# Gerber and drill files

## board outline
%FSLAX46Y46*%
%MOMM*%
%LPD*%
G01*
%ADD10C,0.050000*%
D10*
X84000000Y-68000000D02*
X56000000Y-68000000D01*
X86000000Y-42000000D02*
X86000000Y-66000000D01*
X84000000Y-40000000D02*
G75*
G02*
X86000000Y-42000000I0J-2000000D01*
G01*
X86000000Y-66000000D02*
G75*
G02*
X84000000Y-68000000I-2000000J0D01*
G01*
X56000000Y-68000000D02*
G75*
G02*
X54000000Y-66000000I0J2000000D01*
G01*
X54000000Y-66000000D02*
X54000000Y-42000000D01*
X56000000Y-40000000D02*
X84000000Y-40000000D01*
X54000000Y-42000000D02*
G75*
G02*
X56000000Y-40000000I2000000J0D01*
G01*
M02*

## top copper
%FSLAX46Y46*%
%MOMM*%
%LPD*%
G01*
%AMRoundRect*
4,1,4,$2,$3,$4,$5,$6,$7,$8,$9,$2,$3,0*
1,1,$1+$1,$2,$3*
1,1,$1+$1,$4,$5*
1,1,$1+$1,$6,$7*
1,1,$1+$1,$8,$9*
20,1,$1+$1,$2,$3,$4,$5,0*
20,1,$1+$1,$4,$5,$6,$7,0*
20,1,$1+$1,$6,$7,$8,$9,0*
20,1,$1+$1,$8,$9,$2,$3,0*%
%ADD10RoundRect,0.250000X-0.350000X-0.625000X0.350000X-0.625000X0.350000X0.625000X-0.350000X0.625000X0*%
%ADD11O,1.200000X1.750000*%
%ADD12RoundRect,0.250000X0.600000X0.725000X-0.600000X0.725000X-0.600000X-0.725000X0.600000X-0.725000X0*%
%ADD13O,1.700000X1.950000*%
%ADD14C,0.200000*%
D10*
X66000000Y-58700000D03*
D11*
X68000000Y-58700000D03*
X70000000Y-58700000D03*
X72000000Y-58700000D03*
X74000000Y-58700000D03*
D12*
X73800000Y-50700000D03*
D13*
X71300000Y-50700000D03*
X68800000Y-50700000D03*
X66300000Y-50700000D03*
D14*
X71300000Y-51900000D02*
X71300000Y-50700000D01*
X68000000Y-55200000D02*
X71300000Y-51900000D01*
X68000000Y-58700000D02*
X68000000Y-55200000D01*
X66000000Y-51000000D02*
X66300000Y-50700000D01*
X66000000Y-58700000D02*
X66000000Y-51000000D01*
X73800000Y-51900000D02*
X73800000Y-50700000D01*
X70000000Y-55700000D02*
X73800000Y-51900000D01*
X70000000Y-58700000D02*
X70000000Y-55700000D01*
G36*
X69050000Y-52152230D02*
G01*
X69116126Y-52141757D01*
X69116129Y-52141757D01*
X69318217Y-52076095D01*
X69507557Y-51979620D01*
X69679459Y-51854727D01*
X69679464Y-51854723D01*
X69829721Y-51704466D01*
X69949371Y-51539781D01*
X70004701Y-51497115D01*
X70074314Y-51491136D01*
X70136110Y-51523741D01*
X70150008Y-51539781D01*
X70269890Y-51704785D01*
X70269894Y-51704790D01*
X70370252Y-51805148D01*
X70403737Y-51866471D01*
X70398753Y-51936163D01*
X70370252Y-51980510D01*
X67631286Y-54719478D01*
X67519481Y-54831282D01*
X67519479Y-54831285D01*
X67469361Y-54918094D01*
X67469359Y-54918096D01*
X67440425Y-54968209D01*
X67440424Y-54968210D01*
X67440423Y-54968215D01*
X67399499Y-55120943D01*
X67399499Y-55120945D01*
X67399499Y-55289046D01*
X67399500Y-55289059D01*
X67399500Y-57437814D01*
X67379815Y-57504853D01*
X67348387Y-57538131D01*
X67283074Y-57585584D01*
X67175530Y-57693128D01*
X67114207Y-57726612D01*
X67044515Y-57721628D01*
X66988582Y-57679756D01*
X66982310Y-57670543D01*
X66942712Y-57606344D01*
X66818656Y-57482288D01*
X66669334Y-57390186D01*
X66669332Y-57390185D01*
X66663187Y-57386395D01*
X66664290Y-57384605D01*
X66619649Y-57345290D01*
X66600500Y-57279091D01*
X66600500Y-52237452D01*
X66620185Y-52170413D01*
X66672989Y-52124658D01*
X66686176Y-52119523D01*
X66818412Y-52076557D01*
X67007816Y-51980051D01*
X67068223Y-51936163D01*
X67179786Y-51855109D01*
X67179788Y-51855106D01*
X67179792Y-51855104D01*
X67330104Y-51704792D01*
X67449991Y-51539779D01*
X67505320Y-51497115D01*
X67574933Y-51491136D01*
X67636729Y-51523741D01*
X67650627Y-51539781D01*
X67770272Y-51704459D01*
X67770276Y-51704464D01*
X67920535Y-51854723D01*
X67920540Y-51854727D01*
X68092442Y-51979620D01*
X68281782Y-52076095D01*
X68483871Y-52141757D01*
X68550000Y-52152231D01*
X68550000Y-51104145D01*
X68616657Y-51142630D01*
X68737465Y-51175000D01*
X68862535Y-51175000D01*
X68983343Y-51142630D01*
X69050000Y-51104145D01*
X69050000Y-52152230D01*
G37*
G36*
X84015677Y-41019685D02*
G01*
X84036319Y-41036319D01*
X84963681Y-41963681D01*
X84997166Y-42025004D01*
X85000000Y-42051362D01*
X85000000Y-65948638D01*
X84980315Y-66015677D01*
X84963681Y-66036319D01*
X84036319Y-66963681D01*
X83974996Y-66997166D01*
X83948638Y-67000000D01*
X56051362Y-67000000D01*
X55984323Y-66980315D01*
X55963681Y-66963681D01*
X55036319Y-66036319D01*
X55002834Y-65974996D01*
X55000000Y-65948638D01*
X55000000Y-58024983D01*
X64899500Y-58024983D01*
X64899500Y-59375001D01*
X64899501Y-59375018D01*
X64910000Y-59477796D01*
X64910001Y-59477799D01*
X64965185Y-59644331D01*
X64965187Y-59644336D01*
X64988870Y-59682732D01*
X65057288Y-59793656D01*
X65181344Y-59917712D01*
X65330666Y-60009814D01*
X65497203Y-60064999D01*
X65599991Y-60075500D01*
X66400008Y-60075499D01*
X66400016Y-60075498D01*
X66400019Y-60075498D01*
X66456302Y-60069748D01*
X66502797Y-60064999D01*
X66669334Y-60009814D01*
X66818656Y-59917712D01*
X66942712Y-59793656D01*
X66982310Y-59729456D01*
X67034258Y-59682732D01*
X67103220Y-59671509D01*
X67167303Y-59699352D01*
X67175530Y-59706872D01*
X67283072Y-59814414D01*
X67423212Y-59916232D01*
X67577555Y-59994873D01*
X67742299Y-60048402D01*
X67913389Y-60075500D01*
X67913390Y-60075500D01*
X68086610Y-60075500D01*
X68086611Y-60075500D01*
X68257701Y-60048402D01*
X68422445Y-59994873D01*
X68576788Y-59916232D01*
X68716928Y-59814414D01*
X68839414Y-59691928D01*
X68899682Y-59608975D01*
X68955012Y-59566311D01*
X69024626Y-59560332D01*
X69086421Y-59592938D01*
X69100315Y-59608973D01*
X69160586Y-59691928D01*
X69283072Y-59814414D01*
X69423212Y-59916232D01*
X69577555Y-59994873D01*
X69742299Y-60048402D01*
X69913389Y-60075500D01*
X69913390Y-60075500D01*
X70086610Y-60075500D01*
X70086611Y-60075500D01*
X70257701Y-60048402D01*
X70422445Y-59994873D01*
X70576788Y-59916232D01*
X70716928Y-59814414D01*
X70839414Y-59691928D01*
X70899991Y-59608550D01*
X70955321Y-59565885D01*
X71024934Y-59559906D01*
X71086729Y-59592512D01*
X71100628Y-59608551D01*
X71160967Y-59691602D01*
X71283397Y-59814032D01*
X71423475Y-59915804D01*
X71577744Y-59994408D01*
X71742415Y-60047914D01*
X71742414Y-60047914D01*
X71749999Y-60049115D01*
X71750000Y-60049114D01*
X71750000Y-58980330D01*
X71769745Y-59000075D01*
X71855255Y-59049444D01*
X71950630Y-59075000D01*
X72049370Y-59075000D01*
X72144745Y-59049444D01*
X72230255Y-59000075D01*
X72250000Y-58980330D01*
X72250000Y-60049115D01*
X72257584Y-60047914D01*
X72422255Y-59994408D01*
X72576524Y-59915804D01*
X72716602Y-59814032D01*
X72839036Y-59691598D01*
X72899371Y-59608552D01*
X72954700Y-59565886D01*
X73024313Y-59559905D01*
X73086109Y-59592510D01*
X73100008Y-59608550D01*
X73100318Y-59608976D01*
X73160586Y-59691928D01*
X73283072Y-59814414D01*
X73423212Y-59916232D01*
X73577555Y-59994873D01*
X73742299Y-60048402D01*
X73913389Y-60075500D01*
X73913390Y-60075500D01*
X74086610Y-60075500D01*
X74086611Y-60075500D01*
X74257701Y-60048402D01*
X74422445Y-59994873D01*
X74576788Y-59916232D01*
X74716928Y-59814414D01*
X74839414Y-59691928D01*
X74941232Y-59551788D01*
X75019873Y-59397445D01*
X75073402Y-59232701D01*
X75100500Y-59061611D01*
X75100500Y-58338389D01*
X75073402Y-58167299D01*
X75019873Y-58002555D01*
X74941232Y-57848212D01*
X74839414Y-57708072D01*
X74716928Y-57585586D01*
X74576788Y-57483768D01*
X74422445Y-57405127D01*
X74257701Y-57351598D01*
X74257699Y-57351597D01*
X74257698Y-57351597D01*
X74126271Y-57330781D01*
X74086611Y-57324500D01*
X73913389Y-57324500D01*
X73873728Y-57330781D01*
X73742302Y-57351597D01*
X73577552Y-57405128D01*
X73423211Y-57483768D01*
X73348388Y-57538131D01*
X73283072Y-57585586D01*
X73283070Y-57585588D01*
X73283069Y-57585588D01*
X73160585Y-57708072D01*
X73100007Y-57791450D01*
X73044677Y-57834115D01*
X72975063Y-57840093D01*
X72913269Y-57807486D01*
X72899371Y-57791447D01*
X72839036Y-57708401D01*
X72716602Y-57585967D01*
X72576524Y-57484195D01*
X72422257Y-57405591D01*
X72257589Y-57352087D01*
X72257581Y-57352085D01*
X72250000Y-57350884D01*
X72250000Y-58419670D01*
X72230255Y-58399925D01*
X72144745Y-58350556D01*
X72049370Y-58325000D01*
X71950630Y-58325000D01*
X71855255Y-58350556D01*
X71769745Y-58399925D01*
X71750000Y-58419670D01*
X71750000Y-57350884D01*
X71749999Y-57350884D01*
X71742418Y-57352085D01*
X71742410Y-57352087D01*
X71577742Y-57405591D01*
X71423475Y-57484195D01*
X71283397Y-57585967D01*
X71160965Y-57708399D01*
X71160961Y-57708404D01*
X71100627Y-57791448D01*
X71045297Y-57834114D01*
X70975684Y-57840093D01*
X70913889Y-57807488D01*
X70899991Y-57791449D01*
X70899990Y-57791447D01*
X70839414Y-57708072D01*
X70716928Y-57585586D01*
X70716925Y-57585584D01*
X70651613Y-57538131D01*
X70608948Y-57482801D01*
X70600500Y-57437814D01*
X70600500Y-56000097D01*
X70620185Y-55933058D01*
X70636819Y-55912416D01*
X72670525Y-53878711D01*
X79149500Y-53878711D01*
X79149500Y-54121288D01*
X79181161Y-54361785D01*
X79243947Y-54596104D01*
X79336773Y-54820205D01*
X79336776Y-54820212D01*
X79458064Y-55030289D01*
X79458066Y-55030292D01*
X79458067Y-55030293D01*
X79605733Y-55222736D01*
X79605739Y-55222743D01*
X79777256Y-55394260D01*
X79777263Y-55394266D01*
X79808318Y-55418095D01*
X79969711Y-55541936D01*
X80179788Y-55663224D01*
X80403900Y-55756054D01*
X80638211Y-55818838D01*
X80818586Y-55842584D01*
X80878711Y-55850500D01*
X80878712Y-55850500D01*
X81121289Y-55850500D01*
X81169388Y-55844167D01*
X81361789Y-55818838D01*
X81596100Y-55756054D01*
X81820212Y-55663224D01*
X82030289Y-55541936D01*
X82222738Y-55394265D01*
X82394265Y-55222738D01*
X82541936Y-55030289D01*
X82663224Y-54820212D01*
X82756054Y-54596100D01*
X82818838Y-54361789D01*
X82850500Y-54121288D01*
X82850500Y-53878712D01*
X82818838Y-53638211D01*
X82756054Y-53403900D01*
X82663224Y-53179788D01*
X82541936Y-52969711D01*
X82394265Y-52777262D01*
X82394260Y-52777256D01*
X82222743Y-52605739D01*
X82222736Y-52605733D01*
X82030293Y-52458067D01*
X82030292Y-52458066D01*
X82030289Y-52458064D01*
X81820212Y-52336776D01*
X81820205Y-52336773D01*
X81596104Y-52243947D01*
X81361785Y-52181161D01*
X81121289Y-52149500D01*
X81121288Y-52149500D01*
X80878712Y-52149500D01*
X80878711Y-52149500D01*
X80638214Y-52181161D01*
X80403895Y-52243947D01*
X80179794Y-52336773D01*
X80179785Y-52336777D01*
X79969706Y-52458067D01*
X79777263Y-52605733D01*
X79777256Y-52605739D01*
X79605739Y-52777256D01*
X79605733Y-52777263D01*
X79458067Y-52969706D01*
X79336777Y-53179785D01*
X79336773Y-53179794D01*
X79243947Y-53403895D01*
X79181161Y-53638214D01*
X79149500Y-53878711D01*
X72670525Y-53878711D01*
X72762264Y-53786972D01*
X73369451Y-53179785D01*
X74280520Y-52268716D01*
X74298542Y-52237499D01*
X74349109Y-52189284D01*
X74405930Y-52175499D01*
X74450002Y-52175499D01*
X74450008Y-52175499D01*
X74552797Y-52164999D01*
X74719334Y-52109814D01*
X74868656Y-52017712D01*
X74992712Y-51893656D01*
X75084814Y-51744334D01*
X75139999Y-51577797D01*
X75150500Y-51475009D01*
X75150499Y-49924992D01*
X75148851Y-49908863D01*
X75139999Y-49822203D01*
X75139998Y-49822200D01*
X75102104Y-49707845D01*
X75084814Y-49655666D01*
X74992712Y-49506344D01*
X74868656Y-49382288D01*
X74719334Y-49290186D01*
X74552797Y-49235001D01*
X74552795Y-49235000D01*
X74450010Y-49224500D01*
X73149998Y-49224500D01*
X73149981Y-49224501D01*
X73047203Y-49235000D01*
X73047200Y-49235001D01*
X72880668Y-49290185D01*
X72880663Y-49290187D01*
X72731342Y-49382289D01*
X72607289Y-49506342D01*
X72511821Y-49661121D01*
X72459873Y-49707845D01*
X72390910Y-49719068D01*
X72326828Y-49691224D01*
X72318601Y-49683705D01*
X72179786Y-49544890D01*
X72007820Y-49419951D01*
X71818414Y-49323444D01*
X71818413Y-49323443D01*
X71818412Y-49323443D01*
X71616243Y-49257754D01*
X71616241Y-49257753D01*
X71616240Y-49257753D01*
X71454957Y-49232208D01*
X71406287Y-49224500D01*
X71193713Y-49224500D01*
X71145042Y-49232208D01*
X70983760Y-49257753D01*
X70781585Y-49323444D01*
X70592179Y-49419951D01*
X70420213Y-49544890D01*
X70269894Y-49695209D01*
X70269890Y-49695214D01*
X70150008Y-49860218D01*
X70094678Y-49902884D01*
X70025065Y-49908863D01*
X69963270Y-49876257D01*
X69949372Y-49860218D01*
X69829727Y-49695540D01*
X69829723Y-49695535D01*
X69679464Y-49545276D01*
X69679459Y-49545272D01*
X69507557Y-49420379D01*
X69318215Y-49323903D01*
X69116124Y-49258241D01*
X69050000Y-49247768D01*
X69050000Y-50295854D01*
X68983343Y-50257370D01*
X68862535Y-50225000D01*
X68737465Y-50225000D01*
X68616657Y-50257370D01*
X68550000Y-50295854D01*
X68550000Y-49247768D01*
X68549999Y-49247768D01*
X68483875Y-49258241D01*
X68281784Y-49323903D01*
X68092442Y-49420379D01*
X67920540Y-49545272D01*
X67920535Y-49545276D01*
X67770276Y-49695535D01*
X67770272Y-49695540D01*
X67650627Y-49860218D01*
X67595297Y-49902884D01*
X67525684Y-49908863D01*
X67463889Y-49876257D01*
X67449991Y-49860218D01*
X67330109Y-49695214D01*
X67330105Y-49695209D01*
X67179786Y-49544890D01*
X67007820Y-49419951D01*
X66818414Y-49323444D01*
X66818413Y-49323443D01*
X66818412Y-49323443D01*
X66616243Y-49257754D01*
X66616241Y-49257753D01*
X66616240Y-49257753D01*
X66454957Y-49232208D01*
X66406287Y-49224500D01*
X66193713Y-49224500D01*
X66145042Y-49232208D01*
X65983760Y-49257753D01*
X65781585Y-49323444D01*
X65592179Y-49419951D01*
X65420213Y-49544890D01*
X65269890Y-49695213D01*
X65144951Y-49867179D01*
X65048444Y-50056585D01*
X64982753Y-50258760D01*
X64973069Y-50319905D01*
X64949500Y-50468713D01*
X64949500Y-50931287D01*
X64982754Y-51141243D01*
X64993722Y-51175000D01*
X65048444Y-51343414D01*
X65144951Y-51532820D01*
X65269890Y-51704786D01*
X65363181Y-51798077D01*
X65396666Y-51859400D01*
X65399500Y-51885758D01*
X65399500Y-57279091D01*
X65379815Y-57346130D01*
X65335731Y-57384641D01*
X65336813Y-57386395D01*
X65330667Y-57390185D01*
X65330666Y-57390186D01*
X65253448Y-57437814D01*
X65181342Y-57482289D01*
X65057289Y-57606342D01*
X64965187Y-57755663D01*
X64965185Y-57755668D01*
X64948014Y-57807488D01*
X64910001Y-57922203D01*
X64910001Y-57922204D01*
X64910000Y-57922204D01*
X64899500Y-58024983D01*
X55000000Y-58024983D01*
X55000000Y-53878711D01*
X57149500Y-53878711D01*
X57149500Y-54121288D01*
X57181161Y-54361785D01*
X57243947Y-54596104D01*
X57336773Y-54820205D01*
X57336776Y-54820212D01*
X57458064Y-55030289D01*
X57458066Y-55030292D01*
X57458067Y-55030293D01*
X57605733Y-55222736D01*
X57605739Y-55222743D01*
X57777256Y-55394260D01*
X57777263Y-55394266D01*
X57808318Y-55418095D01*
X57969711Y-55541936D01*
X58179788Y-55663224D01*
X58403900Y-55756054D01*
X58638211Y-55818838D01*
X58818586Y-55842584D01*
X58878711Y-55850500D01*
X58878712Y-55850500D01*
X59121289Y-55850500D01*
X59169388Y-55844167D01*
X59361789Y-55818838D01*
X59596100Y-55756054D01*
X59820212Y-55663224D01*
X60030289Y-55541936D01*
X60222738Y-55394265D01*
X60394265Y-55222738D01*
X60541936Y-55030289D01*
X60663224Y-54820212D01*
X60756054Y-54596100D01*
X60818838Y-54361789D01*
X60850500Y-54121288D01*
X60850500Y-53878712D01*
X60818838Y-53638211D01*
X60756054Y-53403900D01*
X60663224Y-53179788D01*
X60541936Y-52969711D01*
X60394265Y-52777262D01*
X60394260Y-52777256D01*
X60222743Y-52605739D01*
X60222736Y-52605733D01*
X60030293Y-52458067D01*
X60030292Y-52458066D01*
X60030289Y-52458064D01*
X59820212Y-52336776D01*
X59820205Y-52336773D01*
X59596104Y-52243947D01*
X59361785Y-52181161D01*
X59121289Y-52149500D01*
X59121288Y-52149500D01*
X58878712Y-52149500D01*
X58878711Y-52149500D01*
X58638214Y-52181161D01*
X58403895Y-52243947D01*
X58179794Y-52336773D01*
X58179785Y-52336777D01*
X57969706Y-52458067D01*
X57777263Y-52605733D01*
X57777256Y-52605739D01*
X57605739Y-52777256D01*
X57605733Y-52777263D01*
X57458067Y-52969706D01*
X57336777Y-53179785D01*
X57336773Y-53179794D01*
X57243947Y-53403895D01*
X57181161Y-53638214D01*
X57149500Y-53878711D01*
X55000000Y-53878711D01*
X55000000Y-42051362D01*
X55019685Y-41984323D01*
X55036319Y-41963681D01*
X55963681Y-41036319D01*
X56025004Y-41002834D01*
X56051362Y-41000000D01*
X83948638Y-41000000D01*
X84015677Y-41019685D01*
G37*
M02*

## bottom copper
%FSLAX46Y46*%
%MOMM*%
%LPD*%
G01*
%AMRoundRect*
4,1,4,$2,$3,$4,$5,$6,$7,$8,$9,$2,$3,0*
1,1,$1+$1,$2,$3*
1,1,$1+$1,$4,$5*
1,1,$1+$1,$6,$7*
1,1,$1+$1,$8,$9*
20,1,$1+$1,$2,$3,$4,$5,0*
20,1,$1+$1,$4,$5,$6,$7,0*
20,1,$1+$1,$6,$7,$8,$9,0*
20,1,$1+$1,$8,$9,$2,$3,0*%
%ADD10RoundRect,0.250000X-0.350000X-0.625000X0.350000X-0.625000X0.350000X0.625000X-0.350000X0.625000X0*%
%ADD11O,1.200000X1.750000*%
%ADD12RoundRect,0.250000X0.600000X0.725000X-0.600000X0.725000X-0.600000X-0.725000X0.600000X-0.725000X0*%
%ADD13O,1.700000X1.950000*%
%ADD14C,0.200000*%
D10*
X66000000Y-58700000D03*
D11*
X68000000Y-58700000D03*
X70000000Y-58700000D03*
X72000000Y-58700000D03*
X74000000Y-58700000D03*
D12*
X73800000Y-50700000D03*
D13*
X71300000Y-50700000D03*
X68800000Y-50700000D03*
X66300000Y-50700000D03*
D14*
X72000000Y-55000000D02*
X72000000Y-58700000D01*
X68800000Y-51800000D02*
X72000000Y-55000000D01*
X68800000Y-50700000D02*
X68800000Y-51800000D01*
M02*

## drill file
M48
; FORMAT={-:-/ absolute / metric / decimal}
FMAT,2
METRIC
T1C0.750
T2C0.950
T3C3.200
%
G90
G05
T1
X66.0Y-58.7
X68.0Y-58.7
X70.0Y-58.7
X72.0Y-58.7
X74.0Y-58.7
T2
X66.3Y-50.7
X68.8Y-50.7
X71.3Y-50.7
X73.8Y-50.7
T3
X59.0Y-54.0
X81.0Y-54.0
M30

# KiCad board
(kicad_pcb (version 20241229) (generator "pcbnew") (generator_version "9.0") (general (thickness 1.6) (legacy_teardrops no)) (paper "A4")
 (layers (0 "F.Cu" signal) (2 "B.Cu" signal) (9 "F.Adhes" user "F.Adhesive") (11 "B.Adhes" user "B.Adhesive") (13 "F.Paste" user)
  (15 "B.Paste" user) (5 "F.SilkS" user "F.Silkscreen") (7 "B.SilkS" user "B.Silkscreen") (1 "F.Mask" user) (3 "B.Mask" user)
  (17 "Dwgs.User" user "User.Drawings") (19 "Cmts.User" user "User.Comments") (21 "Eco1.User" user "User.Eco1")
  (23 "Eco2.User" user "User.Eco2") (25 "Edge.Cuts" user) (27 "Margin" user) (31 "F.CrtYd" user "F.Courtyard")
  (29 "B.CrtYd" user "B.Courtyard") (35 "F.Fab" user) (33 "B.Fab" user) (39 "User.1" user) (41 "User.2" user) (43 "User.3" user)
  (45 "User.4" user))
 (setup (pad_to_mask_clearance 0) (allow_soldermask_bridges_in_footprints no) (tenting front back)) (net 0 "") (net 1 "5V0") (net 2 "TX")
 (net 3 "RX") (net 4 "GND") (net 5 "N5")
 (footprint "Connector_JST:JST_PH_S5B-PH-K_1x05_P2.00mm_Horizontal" (layer "F.Cu") (at 66 58.7)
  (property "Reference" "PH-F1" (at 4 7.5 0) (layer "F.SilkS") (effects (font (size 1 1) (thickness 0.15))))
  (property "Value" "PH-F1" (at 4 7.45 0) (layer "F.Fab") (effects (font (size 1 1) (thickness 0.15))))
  (pad "1" thru_hole roundrect (at 0 0) (size 1.2 1.75) (drill 0.75) (layers "*.Cu" "*.Mask") (remove_unused_layers no)
   (roundrect_rratio 0.208333) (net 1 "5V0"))
  (pad "2" thru_hole oval (at 2 0) (size 1.2 1.75) (drill 0.75) (layers "*.Cu" "*.Mask") (remove_unused_layers no) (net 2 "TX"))
  (pad "3" thru_hole oval (at 4 0) (size 1.2 1.75) (drill 0.75) (layers "*.Cu" "*.Mask") (remove_unused_layers no) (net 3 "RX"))
  (pad "4" thru_hole oval (at 6 0) (size 1.2 1.75) (drill 0.75) (layers "*.Cu" "*.Mask") (remove_unused_layers no) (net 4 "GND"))
  (pad "5" thru_hole oval (at 8 0) (size 1.2 1.75) (drill 0.75) (layers "*.Cu" "*.Mask") (remove_unused_layers no) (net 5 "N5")))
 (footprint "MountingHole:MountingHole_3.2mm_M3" (layer "F.Cu") (at 59 54)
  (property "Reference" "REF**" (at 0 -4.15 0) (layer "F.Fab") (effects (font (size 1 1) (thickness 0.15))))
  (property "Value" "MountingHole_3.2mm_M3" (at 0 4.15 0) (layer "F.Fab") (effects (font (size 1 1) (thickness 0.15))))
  (pad "" np_thru_hole circle (at 0 0) (size 3.2 3.2) (drill 3.2) (layers "*.Cu" "*.Mask")))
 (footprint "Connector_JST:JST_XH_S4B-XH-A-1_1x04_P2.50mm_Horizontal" (layer "F.Cu") (at 73.8 50.7 180)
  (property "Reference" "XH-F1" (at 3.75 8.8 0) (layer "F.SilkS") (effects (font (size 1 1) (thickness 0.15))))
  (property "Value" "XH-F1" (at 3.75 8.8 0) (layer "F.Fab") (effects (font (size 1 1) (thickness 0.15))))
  (pad "1" thru_hole roundrect (at 0 0 180) (size 1.7 1.95) (drill 0.95) (layers "*.Cu" "*.Mask") (remove_unused_layers no)
   (roundrect_rratio 0.147059) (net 3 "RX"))
  (pad "2" thru_hole oval (at 2.5 0 180) (size 1.7 1.95) (drill 0.95) (layers "*.Cu" "*.Mask") (remove_unused_layers no) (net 2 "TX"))
  (pad "3" thru_hole oval (at 5 0 180) (size 1.7 1.95) (drill 0.95) (layers "*.Cu" "*.Mask") (remove_unused_layers no) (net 4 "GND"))
  (pad "4" thru_hole oval (at 7.5 0 180) (size 1.7 1.95) (drill 0.95) (layers "*.Cu" "*.Mask") (remove_unused_layers no) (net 1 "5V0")))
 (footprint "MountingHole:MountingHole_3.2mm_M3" (layer "F.Cu") (at 81 54)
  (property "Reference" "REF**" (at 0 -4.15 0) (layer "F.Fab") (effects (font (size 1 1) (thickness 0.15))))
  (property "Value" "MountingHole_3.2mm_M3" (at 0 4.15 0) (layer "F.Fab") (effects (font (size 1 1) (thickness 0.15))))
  (pad "" np_thru_hole circle (at 0 0) (size 3.2 3.2) (drill 3.2) (layers "*.Cu" "*.Mask")))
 (gr_line (start 84 68) (end 56 68) (stroke (width 0.05) (type default)) (layer "Edge.Cuts"))
 (gr_line (start 86 42) (end 86 66) (stroke (width 0.05) (type default)) (layer "Edge.Cuts"))
 (gr_arc (start 84 40) (mid 85.414214 40.585786) (end 86 42) (stroke (width 0.05) (type default)) (layer "Edge.Cuts"))
 (gr_arc (start 86 66) (mid 85.414214 67.414214) (end 84 68) (stroke (width 0.05) (type default)) (layer "Edge.Cuts"))
 (gr_arc (start 56 68) (mid 54.585786 67.414214) (end 54 66) (stroke (width 0.05) (type default)) (layer "Edge.Cuts"))
 (gr_line (start 54 66) (end 54 42) (stroke (width 0.05) (type default)) (layer "Edge.Cuts"))
 (gr_line (start 56 40) (end 84 40) (stroke (width 0.05) (type default)) (layer "Edge.Cuts"))
 (gr_arc (start 54 42) (mid 54.585786 40.585786) (end 56 40) (stroke (width 0.05) (type default)) (layer "Edge.Cuts"))
 (segment (start 71.3 51.9) (end 71.3 50.7) (width 0.2) (layer "F.Cu") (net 2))
 (segment (start 68 55.2) (end 71.3 51.9) (width 0.2) (layer "F.Cu") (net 2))
 (segment (start 68 58.7) (end 68 55.2) (width 0.2) (layer "F.Cu") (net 2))
 (segment (start 66 51) (end 66.3 50.7) (width 0.2) (layer "F.Cu") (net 1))
 (segment (start 66 58.7) (end 66 51) (width 0.2) (layer "F.Cu") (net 1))
 (segment (start 73.8 51.9) (end 73.8 50.7) (width 0.2) (layer "F.Cu") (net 3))
 (segment (start 70 55.7) (end 73.8 51.9) (width 0.2) (layer "F.Cu") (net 3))
 (segment (start 70 58.7) (end 70 55.7) (width 0.2) (layer "F.Cu") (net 3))
 (segment (start 72 55) (end 72 58.7) (width 0.2) (layer "B.Cu") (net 4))
 (segment (start 68.8 51.8) (end 72 55) (width 0.2) (layer "B.Cu") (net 4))
 (segment (start 68.8 50.7) (end 68.8 51.8) (width 0.2) (layer "B.Cu") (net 4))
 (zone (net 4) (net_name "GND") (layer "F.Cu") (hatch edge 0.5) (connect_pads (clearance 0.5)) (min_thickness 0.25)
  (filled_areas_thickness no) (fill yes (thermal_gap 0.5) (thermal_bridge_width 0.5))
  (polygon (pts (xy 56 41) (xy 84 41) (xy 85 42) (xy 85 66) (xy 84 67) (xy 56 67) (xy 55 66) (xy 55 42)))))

